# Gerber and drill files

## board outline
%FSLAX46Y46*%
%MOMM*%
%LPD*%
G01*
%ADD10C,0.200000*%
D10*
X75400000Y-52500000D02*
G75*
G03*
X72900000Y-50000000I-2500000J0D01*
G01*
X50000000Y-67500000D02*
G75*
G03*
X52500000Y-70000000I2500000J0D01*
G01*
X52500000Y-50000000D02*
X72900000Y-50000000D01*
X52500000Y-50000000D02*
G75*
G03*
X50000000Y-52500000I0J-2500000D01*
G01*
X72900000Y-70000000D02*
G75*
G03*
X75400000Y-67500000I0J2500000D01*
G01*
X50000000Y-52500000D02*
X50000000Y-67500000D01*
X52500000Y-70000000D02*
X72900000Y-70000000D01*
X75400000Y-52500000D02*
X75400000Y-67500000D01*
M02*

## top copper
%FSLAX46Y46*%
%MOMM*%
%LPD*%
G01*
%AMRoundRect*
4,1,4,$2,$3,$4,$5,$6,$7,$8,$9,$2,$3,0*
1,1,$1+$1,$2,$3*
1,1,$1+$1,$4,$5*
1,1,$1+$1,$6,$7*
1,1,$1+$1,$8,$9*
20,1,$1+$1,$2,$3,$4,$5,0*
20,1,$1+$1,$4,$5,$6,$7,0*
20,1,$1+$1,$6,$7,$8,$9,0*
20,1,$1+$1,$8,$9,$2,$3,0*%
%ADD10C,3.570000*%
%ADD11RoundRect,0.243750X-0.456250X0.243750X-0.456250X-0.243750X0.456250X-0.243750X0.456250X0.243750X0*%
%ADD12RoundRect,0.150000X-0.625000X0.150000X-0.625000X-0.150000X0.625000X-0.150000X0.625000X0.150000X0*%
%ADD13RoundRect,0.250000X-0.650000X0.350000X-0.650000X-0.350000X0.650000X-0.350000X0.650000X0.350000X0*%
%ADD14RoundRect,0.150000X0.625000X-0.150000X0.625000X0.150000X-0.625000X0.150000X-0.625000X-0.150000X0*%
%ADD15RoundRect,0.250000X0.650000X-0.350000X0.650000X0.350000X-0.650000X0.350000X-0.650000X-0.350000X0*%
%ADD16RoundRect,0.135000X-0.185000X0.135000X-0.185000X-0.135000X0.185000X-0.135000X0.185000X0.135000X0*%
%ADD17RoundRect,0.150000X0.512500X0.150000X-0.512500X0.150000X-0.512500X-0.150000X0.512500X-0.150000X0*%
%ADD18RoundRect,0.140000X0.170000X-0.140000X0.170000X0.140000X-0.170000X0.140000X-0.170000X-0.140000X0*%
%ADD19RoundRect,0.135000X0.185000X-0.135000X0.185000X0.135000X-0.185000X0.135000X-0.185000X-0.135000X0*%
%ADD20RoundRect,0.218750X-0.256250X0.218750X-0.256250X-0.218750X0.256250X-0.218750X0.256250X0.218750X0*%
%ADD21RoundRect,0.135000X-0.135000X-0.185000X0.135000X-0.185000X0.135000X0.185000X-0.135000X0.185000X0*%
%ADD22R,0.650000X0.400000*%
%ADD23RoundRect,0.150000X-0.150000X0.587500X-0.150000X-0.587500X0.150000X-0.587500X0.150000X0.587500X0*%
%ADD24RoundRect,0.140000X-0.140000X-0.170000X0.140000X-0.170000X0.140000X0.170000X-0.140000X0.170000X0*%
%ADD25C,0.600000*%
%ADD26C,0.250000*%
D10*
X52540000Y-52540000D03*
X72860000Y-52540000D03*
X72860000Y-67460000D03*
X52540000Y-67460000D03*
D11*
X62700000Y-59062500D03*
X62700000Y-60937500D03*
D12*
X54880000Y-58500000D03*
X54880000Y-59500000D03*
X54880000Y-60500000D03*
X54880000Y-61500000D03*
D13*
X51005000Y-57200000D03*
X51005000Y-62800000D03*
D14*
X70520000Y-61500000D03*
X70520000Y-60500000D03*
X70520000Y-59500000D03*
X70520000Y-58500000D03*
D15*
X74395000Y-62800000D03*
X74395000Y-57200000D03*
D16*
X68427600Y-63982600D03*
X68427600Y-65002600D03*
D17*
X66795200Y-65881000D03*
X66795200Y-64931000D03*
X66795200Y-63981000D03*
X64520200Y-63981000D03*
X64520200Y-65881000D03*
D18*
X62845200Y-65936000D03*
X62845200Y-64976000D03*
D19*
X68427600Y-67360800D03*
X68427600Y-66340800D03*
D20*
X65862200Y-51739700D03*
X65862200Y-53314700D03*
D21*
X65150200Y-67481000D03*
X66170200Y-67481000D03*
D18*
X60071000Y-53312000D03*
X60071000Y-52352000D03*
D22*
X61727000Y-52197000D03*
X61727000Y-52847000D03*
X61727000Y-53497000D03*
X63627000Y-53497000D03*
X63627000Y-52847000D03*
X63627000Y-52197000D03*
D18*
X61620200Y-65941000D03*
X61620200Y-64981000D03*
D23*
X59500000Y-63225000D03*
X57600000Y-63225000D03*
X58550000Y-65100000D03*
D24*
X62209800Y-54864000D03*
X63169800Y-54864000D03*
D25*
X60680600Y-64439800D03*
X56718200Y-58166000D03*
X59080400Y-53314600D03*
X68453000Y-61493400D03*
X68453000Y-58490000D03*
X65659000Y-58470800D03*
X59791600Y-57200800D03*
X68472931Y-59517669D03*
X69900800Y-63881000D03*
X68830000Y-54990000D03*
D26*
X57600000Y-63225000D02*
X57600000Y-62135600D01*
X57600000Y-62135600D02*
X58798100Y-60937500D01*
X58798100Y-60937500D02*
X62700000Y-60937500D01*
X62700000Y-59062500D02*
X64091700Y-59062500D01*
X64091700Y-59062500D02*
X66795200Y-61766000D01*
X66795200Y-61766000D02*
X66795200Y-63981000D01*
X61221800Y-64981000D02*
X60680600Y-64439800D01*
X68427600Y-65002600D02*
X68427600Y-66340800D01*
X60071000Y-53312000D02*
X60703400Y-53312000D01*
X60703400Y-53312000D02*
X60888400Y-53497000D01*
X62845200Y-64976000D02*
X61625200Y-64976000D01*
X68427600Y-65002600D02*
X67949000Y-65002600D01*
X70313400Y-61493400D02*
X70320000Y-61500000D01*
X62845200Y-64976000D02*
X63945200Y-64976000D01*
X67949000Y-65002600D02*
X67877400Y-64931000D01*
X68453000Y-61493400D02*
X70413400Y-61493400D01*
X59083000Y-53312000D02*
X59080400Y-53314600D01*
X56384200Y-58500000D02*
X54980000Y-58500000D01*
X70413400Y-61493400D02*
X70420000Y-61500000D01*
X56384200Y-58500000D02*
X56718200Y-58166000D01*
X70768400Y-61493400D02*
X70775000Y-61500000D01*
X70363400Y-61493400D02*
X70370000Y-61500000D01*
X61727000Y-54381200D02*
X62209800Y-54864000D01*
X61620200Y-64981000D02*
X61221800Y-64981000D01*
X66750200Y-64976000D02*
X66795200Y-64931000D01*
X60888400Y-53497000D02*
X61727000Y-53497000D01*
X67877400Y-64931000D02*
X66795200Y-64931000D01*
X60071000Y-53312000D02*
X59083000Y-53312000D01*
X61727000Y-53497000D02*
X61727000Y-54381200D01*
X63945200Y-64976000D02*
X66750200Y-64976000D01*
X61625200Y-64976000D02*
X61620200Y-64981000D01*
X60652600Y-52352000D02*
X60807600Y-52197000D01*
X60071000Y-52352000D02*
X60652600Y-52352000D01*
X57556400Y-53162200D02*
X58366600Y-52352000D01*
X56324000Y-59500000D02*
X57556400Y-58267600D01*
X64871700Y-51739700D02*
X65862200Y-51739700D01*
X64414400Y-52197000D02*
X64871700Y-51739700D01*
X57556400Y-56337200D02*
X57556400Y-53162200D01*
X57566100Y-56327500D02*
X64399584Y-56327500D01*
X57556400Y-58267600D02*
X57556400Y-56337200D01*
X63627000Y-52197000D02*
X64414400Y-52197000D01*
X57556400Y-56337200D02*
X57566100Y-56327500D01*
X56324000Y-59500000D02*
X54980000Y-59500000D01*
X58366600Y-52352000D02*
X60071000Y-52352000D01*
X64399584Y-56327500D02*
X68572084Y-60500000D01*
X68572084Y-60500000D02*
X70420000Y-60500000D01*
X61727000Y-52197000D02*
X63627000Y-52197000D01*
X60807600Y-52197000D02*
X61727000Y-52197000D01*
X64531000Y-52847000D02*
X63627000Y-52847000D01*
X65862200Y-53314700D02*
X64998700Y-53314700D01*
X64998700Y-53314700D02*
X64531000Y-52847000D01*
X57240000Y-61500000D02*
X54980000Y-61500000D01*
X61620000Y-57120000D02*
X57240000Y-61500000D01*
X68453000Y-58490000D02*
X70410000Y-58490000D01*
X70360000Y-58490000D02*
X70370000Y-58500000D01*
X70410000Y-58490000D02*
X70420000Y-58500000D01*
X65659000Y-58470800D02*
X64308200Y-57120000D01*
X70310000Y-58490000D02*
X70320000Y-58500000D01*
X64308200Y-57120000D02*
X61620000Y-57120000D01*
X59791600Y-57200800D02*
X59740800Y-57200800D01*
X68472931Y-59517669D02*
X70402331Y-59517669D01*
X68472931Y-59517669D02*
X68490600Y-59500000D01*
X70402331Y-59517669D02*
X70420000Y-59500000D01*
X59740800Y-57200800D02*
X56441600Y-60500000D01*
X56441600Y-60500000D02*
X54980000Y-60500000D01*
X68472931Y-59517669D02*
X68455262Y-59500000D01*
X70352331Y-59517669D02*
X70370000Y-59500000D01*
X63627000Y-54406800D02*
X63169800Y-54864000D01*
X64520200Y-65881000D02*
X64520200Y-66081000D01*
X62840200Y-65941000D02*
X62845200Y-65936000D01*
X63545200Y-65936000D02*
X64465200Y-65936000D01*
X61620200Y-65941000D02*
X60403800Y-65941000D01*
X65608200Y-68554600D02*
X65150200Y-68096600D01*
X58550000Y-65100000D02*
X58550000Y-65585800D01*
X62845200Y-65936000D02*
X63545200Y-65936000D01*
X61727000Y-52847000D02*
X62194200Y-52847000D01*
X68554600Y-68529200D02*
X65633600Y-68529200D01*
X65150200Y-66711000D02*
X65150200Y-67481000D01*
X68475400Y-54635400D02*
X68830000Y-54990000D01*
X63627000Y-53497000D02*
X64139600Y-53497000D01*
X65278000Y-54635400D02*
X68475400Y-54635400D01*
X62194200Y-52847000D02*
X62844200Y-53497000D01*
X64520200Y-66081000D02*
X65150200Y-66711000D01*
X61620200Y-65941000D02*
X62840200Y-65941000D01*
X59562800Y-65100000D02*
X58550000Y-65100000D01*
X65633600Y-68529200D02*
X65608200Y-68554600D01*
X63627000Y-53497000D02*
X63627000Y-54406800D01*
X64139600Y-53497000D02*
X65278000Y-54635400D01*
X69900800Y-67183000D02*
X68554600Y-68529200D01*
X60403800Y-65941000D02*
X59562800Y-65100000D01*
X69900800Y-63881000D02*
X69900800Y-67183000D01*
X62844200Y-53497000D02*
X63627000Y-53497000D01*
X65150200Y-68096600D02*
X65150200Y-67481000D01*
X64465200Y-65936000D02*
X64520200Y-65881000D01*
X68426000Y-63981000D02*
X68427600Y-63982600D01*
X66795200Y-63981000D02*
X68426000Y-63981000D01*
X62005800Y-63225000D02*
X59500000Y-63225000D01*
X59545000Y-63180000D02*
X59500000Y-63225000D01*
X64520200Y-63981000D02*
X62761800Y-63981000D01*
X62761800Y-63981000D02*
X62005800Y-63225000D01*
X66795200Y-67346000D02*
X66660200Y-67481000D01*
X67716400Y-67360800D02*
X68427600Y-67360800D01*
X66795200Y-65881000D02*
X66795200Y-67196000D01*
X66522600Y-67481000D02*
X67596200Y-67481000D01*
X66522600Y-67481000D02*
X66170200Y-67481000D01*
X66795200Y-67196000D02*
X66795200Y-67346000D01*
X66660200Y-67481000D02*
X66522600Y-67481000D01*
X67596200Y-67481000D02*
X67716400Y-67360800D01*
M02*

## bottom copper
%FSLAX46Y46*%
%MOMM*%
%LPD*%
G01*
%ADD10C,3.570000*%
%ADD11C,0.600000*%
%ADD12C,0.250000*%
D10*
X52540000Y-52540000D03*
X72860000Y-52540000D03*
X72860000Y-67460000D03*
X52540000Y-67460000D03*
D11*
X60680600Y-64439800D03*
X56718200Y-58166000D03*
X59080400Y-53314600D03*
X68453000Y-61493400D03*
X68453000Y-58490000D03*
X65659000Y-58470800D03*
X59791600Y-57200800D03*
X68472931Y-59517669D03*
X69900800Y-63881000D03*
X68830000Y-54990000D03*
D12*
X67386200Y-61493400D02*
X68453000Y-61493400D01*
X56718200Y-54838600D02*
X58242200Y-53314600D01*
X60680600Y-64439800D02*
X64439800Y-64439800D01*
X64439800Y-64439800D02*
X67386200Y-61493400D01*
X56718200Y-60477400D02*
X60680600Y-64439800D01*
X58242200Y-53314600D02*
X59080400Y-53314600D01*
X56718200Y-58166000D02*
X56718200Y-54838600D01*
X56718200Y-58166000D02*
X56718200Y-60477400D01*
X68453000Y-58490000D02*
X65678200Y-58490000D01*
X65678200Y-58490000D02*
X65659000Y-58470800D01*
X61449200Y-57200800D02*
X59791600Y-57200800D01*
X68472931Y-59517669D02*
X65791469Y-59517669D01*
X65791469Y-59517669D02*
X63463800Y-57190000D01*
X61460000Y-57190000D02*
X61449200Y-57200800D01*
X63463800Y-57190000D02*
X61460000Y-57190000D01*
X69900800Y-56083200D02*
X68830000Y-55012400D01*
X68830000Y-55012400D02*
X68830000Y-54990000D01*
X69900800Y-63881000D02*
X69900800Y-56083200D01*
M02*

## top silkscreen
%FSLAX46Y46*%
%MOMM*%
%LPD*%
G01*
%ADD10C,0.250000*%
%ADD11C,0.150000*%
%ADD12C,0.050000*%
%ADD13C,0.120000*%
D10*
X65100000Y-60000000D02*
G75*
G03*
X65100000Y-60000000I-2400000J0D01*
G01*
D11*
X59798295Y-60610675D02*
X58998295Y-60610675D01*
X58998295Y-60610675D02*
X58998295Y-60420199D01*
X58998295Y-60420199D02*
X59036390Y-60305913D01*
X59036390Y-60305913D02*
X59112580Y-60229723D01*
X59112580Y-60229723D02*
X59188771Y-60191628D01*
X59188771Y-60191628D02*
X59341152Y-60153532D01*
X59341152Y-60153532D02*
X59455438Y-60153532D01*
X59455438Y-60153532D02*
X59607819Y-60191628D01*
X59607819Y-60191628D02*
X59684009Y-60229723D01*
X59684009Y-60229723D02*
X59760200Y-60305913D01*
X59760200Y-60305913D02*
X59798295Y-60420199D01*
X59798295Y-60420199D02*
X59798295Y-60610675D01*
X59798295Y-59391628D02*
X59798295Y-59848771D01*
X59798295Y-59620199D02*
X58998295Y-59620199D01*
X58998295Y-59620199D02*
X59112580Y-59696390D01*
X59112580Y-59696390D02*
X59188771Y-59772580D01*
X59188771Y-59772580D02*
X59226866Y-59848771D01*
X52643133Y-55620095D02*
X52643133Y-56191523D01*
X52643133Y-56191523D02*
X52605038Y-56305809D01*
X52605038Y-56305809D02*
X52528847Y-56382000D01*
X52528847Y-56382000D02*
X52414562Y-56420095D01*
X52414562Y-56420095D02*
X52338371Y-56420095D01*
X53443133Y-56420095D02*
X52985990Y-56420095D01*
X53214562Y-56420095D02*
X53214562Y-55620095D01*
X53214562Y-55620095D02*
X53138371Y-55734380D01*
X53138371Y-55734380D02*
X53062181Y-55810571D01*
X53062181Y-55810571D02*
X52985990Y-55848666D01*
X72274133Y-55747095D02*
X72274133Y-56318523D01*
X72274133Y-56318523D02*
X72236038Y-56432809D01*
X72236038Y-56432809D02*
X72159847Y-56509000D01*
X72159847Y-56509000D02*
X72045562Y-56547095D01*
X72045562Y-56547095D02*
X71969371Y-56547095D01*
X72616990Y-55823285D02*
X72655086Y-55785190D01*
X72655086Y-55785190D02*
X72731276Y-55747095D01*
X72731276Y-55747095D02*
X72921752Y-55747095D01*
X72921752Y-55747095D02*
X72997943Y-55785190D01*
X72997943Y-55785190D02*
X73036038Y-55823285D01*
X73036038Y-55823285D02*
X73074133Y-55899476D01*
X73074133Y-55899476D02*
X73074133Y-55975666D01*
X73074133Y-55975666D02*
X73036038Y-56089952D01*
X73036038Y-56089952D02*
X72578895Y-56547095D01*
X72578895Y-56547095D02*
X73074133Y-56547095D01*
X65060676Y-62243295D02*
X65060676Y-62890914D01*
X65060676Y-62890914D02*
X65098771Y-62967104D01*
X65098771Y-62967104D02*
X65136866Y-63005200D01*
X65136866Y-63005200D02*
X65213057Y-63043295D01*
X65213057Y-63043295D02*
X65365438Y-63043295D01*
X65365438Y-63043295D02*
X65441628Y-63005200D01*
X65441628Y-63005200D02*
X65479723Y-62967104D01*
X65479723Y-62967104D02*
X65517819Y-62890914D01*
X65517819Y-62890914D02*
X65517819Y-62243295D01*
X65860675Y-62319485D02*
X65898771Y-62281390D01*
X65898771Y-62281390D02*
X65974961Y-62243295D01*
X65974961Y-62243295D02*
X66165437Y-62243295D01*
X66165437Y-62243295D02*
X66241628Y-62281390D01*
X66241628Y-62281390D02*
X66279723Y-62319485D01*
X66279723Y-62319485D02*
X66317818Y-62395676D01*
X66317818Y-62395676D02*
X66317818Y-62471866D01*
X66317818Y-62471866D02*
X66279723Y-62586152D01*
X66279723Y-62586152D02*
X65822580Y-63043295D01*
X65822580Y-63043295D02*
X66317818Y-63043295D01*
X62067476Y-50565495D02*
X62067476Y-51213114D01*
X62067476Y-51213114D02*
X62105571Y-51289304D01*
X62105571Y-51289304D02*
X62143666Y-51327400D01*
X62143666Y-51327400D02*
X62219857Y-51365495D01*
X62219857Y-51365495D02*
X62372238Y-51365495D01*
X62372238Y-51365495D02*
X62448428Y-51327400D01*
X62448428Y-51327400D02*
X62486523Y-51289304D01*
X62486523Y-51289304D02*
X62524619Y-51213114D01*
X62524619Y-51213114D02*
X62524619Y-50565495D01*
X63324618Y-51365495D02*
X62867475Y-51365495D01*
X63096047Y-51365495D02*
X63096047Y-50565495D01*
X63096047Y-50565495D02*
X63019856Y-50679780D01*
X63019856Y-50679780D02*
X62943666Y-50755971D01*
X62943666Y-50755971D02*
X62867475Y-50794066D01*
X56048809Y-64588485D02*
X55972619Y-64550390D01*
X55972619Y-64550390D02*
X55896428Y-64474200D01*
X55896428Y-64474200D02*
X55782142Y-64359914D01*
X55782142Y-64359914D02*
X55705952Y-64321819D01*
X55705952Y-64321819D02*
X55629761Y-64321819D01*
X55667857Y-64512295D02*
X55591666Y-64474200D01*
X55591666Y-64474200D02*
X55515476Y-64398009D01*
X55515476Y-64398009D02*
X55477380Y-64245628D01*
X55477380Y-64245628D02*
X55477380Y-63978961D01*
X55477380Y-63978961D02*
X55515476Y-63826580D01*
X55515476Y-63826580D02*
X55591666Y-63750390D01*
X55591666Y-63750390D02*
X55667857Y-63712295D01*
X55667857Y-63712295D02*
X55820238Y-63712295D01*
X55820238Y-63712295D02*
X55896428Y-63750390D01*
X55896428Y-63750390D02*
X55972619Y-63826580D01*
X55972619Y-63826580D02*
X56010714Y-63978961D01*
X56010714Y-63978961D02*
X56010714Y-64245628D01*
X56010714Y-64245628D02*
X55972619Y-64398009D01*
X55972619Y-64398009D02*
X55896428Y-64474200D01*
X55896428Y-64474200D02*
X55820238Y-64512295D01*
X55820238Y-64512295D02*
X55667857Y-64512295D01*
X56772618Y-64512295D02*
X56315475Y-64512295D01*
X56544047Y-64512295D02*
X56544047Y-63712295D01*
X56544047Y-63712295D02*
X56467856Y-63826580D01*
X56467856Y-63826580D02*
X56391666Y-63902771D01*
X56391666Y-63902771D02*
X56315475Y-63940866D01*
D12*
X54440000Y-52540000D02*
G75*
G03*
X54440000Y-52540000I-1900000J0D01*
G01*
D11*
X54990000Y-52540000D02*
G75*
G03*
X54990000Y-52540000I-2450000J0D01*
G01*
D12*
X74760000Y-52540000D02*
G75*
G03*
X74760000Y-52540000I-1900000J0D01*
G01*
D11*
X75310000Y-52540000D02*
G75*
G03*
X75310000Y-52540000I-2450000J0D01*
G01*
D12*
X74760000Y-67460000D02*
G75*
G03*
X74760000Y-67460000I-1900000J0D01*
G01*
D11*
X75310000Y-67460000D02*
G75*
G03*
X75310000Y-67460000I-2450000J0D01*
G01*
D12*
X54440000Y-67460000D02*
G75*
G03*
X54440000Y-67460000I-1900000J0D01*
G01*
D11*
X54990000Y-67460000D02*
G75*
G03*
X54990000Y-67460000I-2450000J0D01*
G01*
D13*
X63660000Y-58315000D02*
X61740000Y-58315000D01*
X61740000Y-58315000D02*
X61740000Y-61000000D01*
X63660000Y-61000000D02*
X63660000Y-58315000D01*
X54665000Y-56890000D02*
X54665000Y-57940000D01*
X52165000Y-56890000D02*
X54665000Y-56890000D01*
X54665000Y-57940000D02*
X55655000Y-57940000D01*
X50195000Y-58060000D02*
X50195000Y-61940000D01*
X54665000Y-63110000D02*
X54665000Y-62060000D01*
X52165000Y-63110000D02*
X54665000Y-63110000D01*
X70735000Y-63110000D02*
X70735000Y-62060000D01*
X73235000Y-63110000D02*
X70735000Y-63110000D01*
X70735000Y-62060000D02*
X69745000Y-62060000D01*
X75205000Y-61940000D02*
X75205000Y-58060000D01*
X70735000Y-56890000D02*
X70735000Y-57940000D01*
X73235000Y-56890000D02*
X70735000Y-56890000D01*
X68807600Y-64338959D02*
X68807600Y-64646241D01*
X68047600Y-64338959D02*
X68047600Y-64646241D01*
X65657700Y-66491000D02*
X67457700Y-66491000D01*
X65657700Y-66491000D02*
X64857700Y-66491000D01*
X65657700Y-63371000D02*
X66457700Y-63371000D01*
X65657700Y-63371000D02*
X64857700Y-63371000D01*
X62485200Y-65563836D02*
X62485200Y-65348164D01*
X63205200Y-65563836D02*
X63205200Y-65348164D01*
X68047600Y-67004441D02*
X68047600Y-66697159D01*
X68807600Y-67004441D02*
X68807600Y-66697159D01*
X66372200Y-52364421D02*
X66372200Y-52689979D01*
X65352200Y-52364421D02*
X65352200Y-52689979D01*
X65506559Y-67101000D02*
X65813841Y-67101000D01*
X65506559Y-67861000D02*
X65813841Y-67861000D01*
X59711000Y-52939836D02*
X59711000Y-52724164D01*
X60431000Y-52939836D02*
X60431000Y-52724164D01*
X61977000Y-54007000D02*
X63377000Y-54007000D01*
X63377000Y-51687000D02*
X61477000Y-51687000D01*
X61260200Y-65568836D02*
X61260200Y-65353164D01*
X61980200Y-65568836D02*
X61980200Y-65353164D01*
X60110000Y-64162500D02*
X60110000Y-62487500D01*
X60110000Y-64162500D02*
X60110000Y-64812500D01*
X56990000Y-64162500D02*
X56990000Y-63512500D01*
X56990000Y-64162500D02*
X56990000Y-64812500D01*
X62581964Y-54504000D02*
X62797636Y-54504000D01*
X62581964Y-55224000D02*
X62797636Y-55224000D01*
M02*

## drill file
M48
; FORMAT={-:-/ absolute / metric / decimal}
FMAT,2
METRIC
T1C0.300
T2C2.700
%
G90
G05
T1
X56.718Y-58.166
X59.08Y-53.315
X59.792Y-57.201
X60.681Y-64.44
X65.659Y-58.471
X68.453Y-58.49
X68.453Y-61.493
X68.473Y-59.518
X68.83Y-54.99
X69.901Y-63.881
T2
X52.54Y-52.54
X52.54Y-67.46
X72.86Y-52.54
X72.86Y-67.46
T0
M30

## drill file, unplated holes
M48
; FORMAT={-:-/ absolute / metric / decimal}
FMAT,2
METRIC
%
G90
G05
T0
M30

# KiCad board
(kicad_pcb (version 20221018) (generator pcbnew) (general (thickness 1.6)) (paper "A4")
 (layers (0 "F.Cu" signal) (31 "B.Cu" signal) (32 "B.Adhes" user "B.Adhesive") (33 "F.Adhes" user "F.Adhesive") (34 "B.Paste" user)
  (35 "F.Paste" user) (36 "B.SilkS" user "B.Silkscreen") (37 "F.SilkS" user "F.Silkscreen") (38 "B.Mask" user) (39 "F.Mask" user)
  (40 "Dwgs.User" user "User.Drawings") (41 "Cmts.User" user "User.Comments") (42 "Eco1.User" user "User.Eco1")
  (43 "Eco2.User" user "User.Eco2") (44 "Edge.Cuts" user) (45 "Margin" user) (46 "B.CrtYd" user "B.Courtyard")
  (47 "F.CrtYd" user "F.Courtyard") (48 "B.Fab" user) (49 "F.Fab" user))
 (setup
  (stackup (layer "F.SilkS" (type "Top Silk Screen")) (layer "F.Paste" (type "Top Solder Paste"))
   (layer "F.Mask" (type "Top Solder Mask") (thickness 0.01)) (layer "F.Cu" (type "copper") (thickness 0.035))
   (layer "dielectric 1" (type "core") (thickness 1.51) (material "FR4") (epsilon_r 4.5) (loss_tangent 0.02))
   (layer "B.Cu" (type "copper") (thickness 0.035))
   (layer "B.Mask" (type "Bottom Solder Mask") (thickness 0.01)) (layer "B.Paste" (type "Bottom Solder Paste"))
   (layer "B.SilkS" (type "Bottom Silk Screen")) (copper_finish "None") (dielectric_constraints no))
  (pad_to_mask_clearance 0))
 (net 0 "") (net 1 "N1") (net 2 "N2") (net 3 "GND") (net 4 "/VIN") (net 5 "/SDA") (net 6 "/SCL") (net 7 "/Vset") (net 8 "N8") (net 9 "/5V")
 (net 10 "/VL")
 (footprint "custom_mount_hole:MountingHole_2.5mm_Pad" (layer "F.Cu") (at 52.54 52.54)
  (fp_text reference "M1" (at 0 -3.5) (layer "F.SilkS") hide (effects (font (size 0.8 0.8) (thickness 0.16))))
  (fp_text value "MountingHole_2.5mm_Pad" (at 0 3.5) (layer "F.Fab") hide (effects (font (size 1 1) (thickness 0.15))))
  (fp_circle (center 0 0) (end 1.9 0) (stroke (width 0.05) (type solid)) (fill none) (layer "F.SilkS"))
  (fp_circle (center 0 0) (end 2.45 0) (stroke (width 0.15) (type solid)) (fill none) (layer "F.SilkS"))
  (pad "~" thru_hole circle (at 0 0) (size 3.57 3.57) (drill 2.7) (layers "*.Cu" "*.Mask")))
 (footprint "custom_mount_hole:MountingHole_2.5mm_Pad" (layer "F.Cu") (at 72.86 52.54)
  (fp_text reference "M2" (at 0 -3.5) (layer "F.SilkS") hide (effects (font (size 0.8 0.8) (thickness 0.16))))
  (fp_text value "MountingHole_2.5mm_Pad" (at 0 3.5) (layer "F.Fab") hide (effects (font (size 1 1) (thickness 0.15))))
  (fp_circle (center 0 0) (end 1.9 0) (stroke (width 0.05) (type solid)) (fill none) (layer "F.SilkS"))
  (fp_circle (center 0 0) (end 2.45 0) (stroke (width 0.15) (type solid)) (fill none) (layer "F.SilkS"))
  (pad "~" thru_hole circle (at 0 0) (size 3.57 3.57) (drill 2.7) (layers "*.Cu" "*.Mask")))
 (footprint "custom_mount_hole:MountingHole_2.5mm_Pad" (layer "F.Cu") (at 72.86 67.46)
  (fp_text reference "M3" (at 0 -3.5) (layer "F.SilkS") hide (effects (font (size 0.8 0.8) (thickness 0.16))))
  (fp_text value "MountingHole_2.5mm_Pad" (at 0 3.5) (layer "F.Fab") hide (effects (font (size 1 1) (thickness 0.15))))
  (fp_circle (center 0 0) (end 1.9 0) (stroke (width 0.05) (type solid)) (fill none) (layer "F.SilkS"))
  (fp_circle (center 0 0) (end 2.45 0) (stroke (width 0.15) (type solid)) (fill none) (layer "F.SilkS"))
  (pad "~" thru_hole circle (at 0 0) (size 3.57 3.57) (drill 2.7) (layers "*.Cu" "*.Mask")))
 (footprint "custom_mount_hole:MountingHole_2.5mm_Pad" (layer "F.Cu") (at 52.54 67.46)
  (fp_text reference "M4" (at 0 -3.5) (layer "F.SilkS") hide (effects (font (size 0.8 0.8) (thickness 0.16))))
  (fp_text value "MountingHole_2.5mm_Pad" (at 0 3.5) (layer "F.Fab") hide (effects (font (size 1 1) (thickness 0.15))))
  (fp_circle (center 0 0) (end 1.9 0) (stroke (width 0.05) (type solid)) (fill none) (layer "F.SilkS"))
  (fp_circle (center 0 0) (end 2.45 0) (stroke (width 0.15) (type solid)) (fill none) (layer "F.SilkS"))
  (pad "~" thru_hole circle (at 0 0) (size 3.57 3.57) (drill 2.7) (layers "*.Cu" "*.Mask")))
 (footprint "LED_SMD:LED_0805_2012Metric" (layer "F.Cu") (at 62.7 60 -90)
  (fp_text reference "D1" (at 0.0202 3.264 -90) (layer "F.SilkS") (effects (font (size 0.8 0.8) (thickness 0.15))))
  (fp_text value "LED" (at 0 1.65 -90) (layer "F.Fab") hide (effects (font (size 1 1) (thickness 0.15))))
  (fp_line (start -1.685 -0.96) (end -1.685 0.96) (stroke (width 0.12) (type solid)) (layer "F.SilkS"))
  (fp_line (start -1.685 0.96) (end 1 0.96) (stroke (width 0.12) (type solid)) (layer "F.SilkS"))
  (fp_line (start 1 -0.96) (end -1.685 -0.96) (stroke (width 0.12) (type solid)) (layer "F.SilkS"))
  (pad "1" smd roundrect (at -0.9375 0 270) (size 0.975 1.4) (layers "F.Cu" "F.Paste" "F.Mask") (roundrect_rratio 0.25) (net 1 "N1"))
  (pad "2" smd roundrect (at 0.9375 0 270) (size 0.975 1.4) (layers "F.Cu" "F.Paste" "F.Mask") (roundrect_rratio 0.25) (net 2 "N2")))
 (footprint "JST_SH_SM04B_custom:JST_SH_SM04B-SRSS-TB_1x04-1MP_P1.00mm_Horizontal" (layer "F.Cu") (at 52.88 60 -90)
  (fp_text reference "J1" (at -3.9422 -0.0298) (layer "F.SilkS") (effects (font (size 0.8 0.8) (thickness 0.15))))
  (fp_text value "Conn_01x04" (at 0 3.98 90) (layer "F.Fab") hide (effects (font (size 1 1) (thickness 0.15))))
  (fp_line (start -3.11 -1.785) (end -2.06 -1.785) (stroke (width 0.12) (type solid)) (layer "F.SilkS"))
  (fp_line (start -3.11 0.715) (end -3.11 -1.785) (stroke (width 0.12) (type solid)) (layer "F.SilkS"))
  (fp_line (start -2.06 -1.785) (end -2.06 -2.775) (stroke (width 0.12) (type solid)) (layer "F.SilkS"))
  (fp_line (start -1.94 2.685) (end 1.94 2.685) (stroke (width 0.12) (type solid)) (layer "F.SilkS"))
  (fp_line (start 3.11 -1.785) (end 2.06 -1.785) (stroke (width 0.12) (type solid)) (layer "F.SilkS"))
  (fp_line (start 3.11 0.715) (end 3.11 -1.785) (stroke (width 0.12) (type solid)) (layer "F.SilkS"))
  (pad "1" smd roundrect (at -1.5 -2 270) (size 0.6 1.55) (layers "F.Cu" "F.Paste" "F.Mask") (roundrect_rratio 0.25) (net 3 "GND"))
  (pad "2" smd roundrect (at -0.5 -2 270) (size 0.6 1.55) (layers "F.Cu" "F.Paste" "F.Mask") (roundrect_rratio 0.25) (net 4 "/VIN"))
  (pad "3" smd roundrect (at 0.5 -2 270) (size 0.6 1.55) (layers "F.Cu" "F.Paste" "F.Mask") (roundrect_rratio 0.25) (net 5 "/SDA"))
  (pad "4" smd roundrect (at 1.5 -2 270) (size 0.6 1.55) (layers "F.Cu" "F.Paste" "F.Mask") (roundrect_rratio 0.25) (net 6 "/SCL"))
  (pad "MP" smd roundrect (at -2.8 1.875 270) (size 1.2 1.8) (layers "F.Cu" "F.Paste" "F.Mask") (roundrect_rratio 0.2083333333))
  (pad "MP" smd roundrect (at 2.8 1.875 270) (size 1.2 1.8) (layers "F.Cu" "F.Paste" "F.Mask") (roundrect_rratio 0.2083333333)))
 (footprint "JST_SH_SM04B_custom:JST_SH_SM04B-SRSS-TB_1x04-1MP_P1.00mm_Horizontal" (layer "F.Cu") (at 72.52 60 90)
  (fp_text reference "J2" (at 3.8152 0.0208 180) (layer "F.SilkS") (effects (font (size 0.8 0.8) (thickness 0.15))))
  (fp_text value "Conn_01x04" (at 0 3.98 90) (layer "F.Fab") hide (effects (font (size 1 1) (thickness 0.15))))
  (fp_line (start -3.11 -1.785) (end -2.06 -1.785) (stroke (width 0.12) (type solid)) (layer "F.SilkS"))
  (fp_line (start -3.11 0.715) (end -3.11 -1.785) (stroke (width 0.12) (type solid)) (layer "F.SilkS"))
  (fp_line (start -2.06 -1.785) (end -2.06 -2.775) (stroke (width 0.12) (type solid)) (layer "F.SilkS"))
  (fp_line (start -1.94 2.685) (end 1.94 2.685) (stroke (width 0.12) (type solid)) (layer "F.SilkS"))
  (fp_line (start 3.11 -1.785) (end 2.06 -1.785) (stroke (width 0.12) (type solid)) (layer "F.SilkS"))
  (fp_line (start 3.11 0.715) (end 3.11 -1.785) (stroke (width 0.12) (type solid)) (layer "F.SilkS"))
  (pad "1" smd roundrect (at -1.5 -2 90) (size 0.6 1.55) (layers "F.Cu" "F.Paste" "F.Mask") (roundrect_rratio 0.25) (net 3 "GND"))
  (pad "2" smd roundrect (at -0.5 -2 90) (size 0.6 1.55) (layers "F.Cu" "F.Paste" "F.Mask") (roundrect_rratio 0.25) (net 4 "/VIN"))
  (pad "3" smd roundrect (at 0.5 -2 90) (size 0.6 1.55) (layers "F.Cu" "F.Paste" "F.Mask") (roundrect_rratio 0.25) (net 5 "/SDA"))
  (pad "4" smd roundrect (at 1.5 -2 90) (size 0.6 1.55) (layers "F.Cu" "F.Paste" "F.Mask") (roundrect_rratio 0.25) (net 6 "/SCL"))
  (pad "MP" smd roundrect (at -2.8 1.875 90) (size 1.2 1.8) (layers "F.Cu" "F.Paste" "F.Mask") (roundrect_rratio 0.2083333333))
  (pad "MP" smd roundrect (at 2.8 1.875 90) (size 1.2 1.8) (layers "F.Cu" "F.Paste" "F.Mask") (roundrect_rratio 0.2083333333)))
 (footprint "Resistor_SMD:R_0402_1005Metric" (layer "F.Cu") (at 68.4276 64.4926 -90)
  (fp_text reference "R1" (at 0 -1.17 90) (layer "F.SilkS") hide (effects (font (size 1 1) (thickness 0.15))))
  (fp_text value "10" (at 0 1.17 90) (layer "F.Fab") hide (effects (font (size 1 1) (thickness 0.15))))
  (fp_line (start -0.153641 -0.38) (end 0.153641 -0.38) (stroke (width 0.12) (type solid)) (layer "F.SilkS"))
  (fp_line (start -0.153641 0.38) (end 0.153641 0.38) (stroke (width 0.12) (type solid)) (layer "F.SilkS"))
  (pad "1" smd roundrect (at -0.51 0 270) (size 0.54 0.64) (layers "F.Cu" "F.Paste" "F.Mask") (roundrect_rratio 0.25) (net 1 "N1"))
  (pad "2" smd roundrect (at 0.51 0 270) (size 0.54 0.64) (layers "F.Cu" "F.Paste" "F.Mask") (roundrect_rratio 0.25) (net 3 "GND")))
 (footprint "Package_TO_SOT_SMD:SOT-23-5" (layer "F.Cu") (at 65.6577 64.931 180)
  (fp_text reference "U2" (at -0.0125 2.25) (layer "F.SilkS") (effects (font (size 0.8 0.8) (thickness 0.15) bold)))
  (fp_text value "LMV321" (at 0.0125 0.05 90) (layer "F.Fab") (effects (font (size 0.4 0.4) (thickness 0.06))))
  (fp_line (start 0 -1.56) (end -1.8 -1.56) (stroke (width 0.12) (type solid)) (layer "F.SilkS"))
  (fp_line (start 0 -1.56) (end 0.8 -1.56) (stroke (width 0.12) (type solid)) (layer "F.SilkS"))
  (fp_line (start 0 1.56) (end -0.8 1.56) (stroke (width 0.12) (type solid)) (layer "F.SilkS"))
  (fp_line (start 0 1.56) (end 0.8 1.56) (stroke (width 0.12) (type solid)) (layer "F.SilkS"))
  (pad "1" smd roundrect (at -1.1375 -0.95 180) (size 1.325 0.6) (layers "F.Cu" "F.Paste" "F.Mask") (roundrect_rratio 0.25) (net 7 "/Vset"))
  (pad "2" smd roundrect (at -1.1375 0 180) (size 1.325 0.6) (layers "F.Cu" "F.Paste" "F.Mask") (roundrect_rratio 0.25) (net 3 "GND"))
  (pad "3" smd roundrect (at -1.1375 0.95 180) (size 1.325 0.6) (layers "F.Cu" "F.Paste" "F.Mask") (roundrect_rratio 0.25) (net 1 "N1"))
  (pad "4" smd roundrect (at 1.1375 0.95 180) (size 1.325 0.6) (layers "F.Cu" "F.Paste" "F.Mask") (roundrect_rratio 0.25) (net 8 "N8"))
  (pad "5" smd roundrect (at 1.1375 -0.95 180) (size 1.325 0.6) (layers "F.Cu" "F.Paste" "F.Mask") (roundrect_rratio 0.25) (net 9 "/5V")))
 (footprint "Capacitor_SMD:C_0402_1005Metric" (layer "F.Cu") (at 62.8452 65.456 90)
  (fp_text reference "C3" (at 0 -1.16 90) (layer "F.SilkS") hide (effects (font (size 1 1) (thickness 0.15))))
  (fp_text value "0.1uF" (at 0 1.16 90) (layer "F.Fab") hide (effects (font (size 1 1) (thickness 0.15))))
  (fp_line (start -0.107836 -0.36) (end 0.107836 -0.36) (stroke (width 0.12) (type solid)) (layer "F.SilkS"))
  (fp_line (start -0.107836 0.36) (end 0.107836 0.36) (stroke (width 0.12) (type solid)) (layer "F.SilkS"))
  (pad "1" smd roundrect (at -0.48 0 90) (size 0.56 0.62) (layers "F.Cu" "F.Paste" "F.Mask") (roundrect_rratio 0.25) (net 9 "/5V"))
  (pad "2" smd roundrect (at 0.48 0 90) (size 0.56 0.62) (layers "F.Cu" "F.Paste" "F.Mask") (roundrect_rratio 0.25) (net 3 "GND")))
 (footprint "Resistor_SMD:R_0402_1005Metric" (layer "F.Cu") (at 68.4276 66.8508 90)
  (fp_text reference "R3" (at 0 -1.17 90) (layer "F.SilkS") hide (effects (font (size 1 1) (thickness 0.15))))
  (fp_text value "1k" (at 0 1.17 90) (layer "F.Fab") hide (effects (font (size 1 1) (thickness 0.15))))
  (fp_line (start -0.153641 -0.38) (end 0.153641 -0.38) (stroke (width 0.12) (type solid)) (layer "F.SilkS"))
  (fp_line (start -0.153641 0.38) (end 0.153641 0.38) (stroke (width 0.12) (type solid)) (layer "F.SilkS"))
  (pad "1" smd roundrect (at -0.51 0 90) (size 0.54 0.64) (layers "F.Cu" "F.Paste" "F.Mask") (roundrect_rratio 0.25) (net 7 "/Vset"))
  (pad "2" smd roundrect (at 0.51 0 90) (size 0.54 0.64) (layers "F.Cu" "F.Paste" "F.Mask") (roundrect_rratio 0.25) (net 3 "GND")))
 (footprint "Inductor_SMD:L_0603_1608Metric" (layer "F.Cu") (at 65.8622 52.5272 -90)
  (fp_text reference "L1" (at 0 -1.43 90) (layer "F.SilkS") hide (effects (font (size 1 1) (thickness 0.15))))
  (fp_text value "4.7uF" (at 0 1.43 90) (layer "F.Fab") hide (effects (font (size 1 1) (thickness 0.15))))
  (fp_line (start -0.162779 -0.51) (end 0.162779 -0.51) (stroke (width 0.12) (type solid)) (layer "F.SilkS"))
  (fp_line (start -0.162779 0.51) (end 0.162779 0.51) (stroke (width 0.12) (type solid)) (layer "F.SilkS"))
  (pad "1" smd roundrect (at -0.7875 0 270) (size 0.875 0.95) (layers "F.Cu" "F.Paste" "F.Mask") (roundrect_rratio 0.25) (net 4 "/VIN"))
  (pad "2" smd roundrect (at 0.7875 0 270) (size 0.875 0.95) (layers "F.Cu" "F.Paste" "F.Mask") (roundrect_rratio 0.25) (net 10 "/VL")))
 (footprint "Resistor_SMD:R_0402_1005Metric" (layer "F.Cu") (at 65.6602 67.481)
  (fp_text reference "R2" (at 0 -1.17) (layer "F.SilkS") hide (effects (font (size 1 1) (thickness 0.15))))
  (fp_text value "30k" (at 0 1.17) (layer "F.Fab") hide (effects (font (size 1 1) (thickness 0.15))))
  (fp_line (start -0.153641 -0.38) (end 0.153641 -0.38) (stroke (width 0.12) (type solid)) (layer "F.SilkS"))
  (fp_line (start -0.153641 0.38) (end 0.153641 0.38) (stroke (width 0.12) (type solid)) (layer "F.SilkS"))
  (pad "1" smd roundrect (at -0.51 0) (size 0.54 0.64) (layers "F.Cu" "F.Paste" "F.Mask") (roundrect_rratio 0.25) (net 9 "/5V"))
  (pad "2" smd roundrect (at 0.51 0) (size 0.54 0.64) (layers "F.Cu" "F.Paste" "F.Mask") (roundrect_rratio 0.25) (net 7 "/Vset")))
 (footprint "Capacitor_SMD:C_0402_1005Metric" (layer "F.Cu") (at 60.071 52.832 90)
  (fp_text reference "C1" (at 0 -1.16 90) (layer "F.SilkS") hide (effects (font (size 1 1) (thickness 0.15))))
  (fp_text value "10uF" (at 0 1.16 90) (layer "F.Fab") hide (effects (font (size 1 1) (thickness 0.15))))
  (fp_line (start -0.107836 -0.36) (end 0.107836 -0.36) (stroke (width 0.12) (type solid)) (layer "F.SilkS"))
  (fp_line (start -0.107836 0.36) (end 0.107836 0.36) (stroke (width 0.12) (type solid)) (layer "F.SilkS"))
  (pad "1" smd roundrect (at -0.48 0 90) (size 0.56 0.62) (layers "F.Cu" "F.Paste" "F.Mask") (roundrect_rratio 0.25) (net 3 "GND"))
  (pad "2" smd roundrect (at 0.48 0 90) (size 0.56 0.62) (layers "F.Cu" "F.Paste" "F.Mask") (roundrect_rratio 0.25) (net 4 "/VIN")))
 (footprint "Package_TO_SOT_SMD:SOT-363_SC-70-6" (layer "F.Cu") (at 62.677 52.847)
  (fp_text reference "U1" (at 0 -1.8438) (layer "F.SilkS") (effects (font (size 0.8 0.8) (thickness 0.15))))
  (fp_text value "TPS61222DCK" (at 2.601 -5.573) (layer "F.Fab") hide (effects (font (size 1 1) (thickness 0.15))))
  (fp_line (start -0.7 1.16) (end 0.7 1.16) (stroke (width 0.12) (type solid)) (layer "F.SilkS"))
  (fp_line (start 0.7 -1.16) (end -1.2 -1.16) (stroke (width 0.12) (type solid)) (layer "F.SilkS"))
  (pad "1" smd rect (at -0.95 -0.65) (size 0.65 0.4) (layers "F.Cu" "F.Paste" "F.Mask") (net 4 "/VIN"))
  (pad "2" smd rect (at -0.95 0) (size 0.65 0.4) (layers "F.Cu" "F.Paste" "F.Mask") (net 9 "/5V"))
  (pad "3" smd rect (at -0.95 0.65) (size 0.65 0.4) (layers "F.Cu" "F.Paste" "F.Mask") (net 3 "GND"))
  (pad "4" smd rect (at 0.95 0.65) (size 0.65 0.4) (layers "F.Cu" "F.Paste" "F.Mask") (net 9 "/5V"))
  (pad "5" smd rect (at 0.95 0) (size 0.65 0.4) (layers "F.Cu" "F.Paste" "F.Mask") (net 10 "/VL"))
  (pad "6" smd rect (at 0.95 -0.65) (size 0.65 0.4) (layers "F.Cu" "F.Paste" "F.Mask") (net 4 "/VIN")))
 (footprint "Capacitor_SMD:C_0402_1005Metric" (layer "F.Cu") (at 61.6202 65.461 90)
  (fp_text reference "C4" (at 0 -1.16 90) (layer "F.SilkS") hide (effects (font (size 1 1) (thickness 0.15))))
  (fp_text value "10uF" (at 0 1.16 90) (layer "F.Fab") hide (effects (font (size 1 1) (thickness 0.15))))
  (fp_line (start -0.107836 -0.36) (end 0.107836 -0.36) (stroke (width 0.12) (type solid)) (layer "F.SilkS"))
  (fp_line (start -0.107836 0.36) (end 0.107836 0.36) (stroke (width 0.12) (type solid)) (layer "F.SilkS"))
  (pad "1" smd roundrect (at -0.48 0 90) (size 0.56 0.62) (layers "F.Cu" "F.Paste" "F.Mask") (roundrect_rratio 0.25) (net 9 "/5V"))
  (pad "2" smd roundrect (at 0.48 0 90) (size 0.56 0.62) (layers "F.Cu" "F.Paste" "F.Mask") (roundrect_rratio 0.25) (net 3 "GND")))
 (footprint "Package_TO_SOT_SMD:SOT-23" (layer "F.Cu") (at 58.55 64.1625 -90)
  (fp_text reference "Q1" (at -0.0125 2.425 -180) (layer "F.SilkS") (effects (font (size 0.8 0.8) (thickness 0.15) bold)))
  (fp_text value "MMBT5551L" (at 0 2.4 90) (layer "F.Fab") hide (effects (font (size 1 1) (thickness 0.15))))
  (fp_line (start 0 -1.56) (end -1.675 -1.56) (stroke (width 0.12) (type solid)) (layer "F.SilkS"))
  (fp_line (start 0 -1.56) (end 0.65 -1.56) (stroke (width 0.12) (type solid)) (layer "F.SilkS"))
  (fp_line (start 0 1.56) (end -0.65 1.56) (stroke (width 0.12) (type solid)) (layer "F.SilkS"))
  (fp_line (start 0 1.56) (end 0.65 1.56) (stroke (width 0.12) (type solid)) (layer "F.SilkS"))
  (pad "1" smd roundrect (at -0.9375 -0.95 270) (size 1.475 0.6) (layers "F.Cu" "F.Paste" "F.Mask") (roundrect_rratio 0.25) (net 8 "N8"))
  (pad "2" smd roundrect (at -0.9375 0.95 270) (size 1.475 0.6) (layers "F.Cu" "F.Paste" "F.Mask") (roundrect_rratio 0.25) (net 2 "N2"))
  (pad "3" smd roundrect (at 0.9375 0 270) (size 1.475 0.6) (layers "F.Cu" "F.Paste" "F.Mask") (roundrect_rratio 0.25) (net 9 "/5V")))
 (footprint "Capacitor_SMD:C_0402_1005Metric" (layer "F.Cu") (at 62.6898 54.864)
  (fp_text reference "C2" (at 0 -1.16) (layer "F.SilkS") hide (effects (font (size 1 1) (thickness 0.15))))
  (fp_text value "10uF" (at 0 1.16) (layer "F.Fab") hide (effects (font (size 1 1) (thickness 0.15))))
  (fp_line (start -0.107836 -0.36) (end 0.107836 -0.36) (stroke (width 0.12) (type solid)) (layer "F.SilkS"))
  (fp_line (start -0.107836 0.36) (end 0.107836 0.36) (stroke (width 0.12) (type solid)) (layer "F.SilkS"))
  (pad "1" smd roundrect (at -0.48 0) (size 0.56 0.62) (layers "F.Cu" "F.Paste" "F.Mask") (roundrect_rratio 0.25) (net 3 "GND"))
  (pad "2" smd roundrect (at 0.48 0) (size 0.56 0.62) (layers "F.Cu" "F.Paste" "F.Mask") (roundrect_rratio 0.25) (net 9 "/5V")))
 (gr_circle (center 62.7 60) (end 65.1 60) (stroke (width 0.25) (type solid)) (fill none) (layer "F.SilkS"))
 (gr_arc (start 72.9 50) (mid 74.667767 50.732233) (end 75.4 52.5) (stroke (width 0.2) (type solid)) (layer "Edge.Cuts"))
 (gr_arc (start 52.5 70) (mid 50.732233 69.267767) (end 50 67.5) (stroke (width 0.2) (type solid)) (layer "Edge.Cuts"))
 (gr_line (start 52.5 50) (end 72.9 50) (stroke (width 0.2) (type solid)) (layer "Edge.Cuts"))
 (gr_arc (start 50 52.5) (mid 50.732233 50.732233) (end 52.5 50) (stroke (width 0.2) (type solid)) (layer "Edge.Cuts"))
 (gr_arc (start 75.4 67.5) (mid 74.667767 69.267767) (end 72.9 70) (stroke (width 0.2) (type solid)) (layer "Edge.Cuts"))
 (gr_line (start 50 52.5) (end 50 67.5) (stroke (width 0.2) (type solid)) (layer "Edge.Cuts"))
 (gr_line (start 52.5 70) (end 72.9 70) (stroke (width 0.2) (type solid)) (layer "Edge.Cuts"))
 (gr_line (start 75.4 52.5) (end 75.4 67.5) (stroke (width 0.2) (type solid)) (layer "Edge.Cuts"))
 (segment (start 61.2218 64.981) (end 60.6806 64.4398) (width 0.25) (layer "F.Cu") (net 3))
 (segment (start 68.4276 65.0026) (end 68.4276 66.3408) (width 0.25) (layer "F.Cu") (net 3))
 (segment (start 60.071 53.312) (end 60.7034 53.312) (width 0.25) (layer "F.Cu") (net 3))
 (segment (start 60.7034 53.312) (end 60.8884 53.497) (width 0.25) (layer "F.Cu") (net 3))
 (segment (start 62.8452 64.976) (end 61.6252 64.976) (width 0.25) (layer "F.Cu") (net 3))
 (segment (start 68.4276 65.0026) (end 67.949 65.0026) (width 0.25) (layer "F.Cu") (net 3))
 (segment (start 70.3134 61.4934) (end 70.32 61.5) (width 0.25) (layer "F.Cu") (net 3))
 (segment (start 62.8452 64.976) (end 63.9452 64.976) (width 0.25) (layer "F.Cu") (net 3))
 (segment (start 67.949 65.0026) (end 67.8774 64.931) (width 0.25) (layer "F.Cu") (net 3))
 (segment (start 68.453 61.4934) (end 70.4134 61.4934) (width 0.25) (layer "F.Cu") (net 3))
 (segment (start 59.083 53.312) (end 59.0804 53.3146) (width 0.25) (layer "F.Cu") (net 3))
 (segment (start 56.3842 58.5) (end 54.98 58.5) (width 0.25) (layer "F.Cu") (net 3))
 (segment (start 70.4134 61.4934) (end 70.42 61.5) (width 0.25) (layer "F.Cu") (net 3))
 (segment (start 56.3842 58.5) (end 56.7182 58.166) (width 0.25) (layer "F.Cu") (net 3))
 (segment (start 70.7684 61.4934) (end 70.775 61.5) (width 0.25) (layer "F.Cu") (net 3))
 (segment (start 70.3634 61.4934) (end 70.37 61.5) (width 0.25) (layer "F.Cu") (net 3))
 (segment (start 61.727 54.3812) (end 62.2098 54.864) (width 0.25) (layer "F.Cu") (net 3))
 (segment (start 61.6202 64.981) (end 61.2218 64.981) (width 0.25) (layer "F.Cu") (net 3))
 (segment (start 66.7502 64.976) (end 66.7952 64.931) (width 0.25) (layer "F.Cu") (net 3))
 (segment (start 60.8884 53.497) (end 61.727 53.497) (width 0.25) (layer "F.Cu") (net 3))
 (segment (start 67.8774 64.931) (end 66.7952 64.931) (width 0.25) (layer "F.Cu") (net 3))
 (segment (start 60.071 53.312) (end 59.083 53.312) (width 0.25) (layer "F.Cu") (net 3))
 (segment (start 61.727 53.497) (end 61.727 54.3812) (width 0.25) (layer "F.Cu") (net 3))
 (segment (start 63.9452 64.976) (end 66.7502 64.976) (width 0.25) (layer "F.Cu") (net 3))
 (segment (start 61.6252 64.976) (end 61.6202 64.981) (width 0.25) (layer "F.Cu") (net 3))
 (via (at 60.6806 64.4398) (size 0.6) (drill 0.3) (layers "F.Cu" "B.Cu") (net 3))
 (via (at 56.7182 58.166) (size 0.6) (drill 0.3) (layers "F.Cu" "B.Cu") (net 3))
 (via (at 59.0804 53.3146) (size 0.6) (drill 0.3) (layers "F.Cu" "B.Cu") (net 3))
 (via (at 68.453 61.4934) (size 0.6) (drill 0.3) (layers "F.Cu" "B.Cu") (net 3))
 (segment (start 67.3862 61.4934) (end 68.453 61.4934) (width 0.25) (layer "B.Cu") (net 3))
 (segment (start 56.7182 54.8386) (end 58.2422 53.3146) (width 0.25) (layer "B.Cu") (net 3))
 (segment (start 60.6806 64.4398) (end 64.4398 64.4398) (width 0.25) (layer "B.Cu") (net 3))
 (segment (start 64.4398 64.4398) (end 67.3862 61.4934) (width 0.25) (layer "B.Cu") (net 3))
 (segment (start 56.7182 60.4774) (end 60.6806 64.4398) (width 0.25) (layer "B.Cu") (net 3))
 (segment (start 58.2422 53.3146) (end 59.0804 53.3146) (width 0.25) (layer "B.Cu") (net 3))
 (segment (start 56.7182 58.166) (end 56.7182 54.8386) (width 0.25) (layer "B.Cu") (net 3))
 (segment (start 56.7182 58.166) (end 56.7182 60.4774) (width 0.25) (layer "B.Cu") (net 3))
 (segment (start 60.6526 52.352) (end 60.8076 52.197) (width 0.25) (layer "F.Cu") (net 4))
 (segment (start 60.071 52.352) (end 60.6526 52.352) (width 0.25) (layer "F.Cu") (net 4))
 (segment (start 57.5564 53.1622) (end 58.3666 52.352) (width 0.25) (layer "F.Cu") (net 4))
 (segment (start 56.324 59.5) (end 57.5564 58.2676) (width 0.25) (layer "F.Cu") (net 4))
 (segment (start 64.8717 51.7397) (end 65.8622 51.7397) (width 0.25) (layer "F.Cu") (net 4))
 (segment (start 64.4144 52.197) (end 64.8717 51.7397) (width 0.25) (layer "F.Cu") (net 4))
 (segment (start 57.5564 56.3372) (end 57.5564 53.1622) (width 0.25) (layer "F.Cu") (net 4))
 (segment (start 57.5661 56.3275) (end 64.399584 56.3275) (width 0.25) (layer "F.Cu") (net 4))
 (segment (start 57.5564 58.2676) (end 57.5564 56.3372) (width 0.25) (layer "F.Cu") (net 4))
 (segment (start 63.627 52.197) (end 64.4144 52.197) (width 0.25) (layer "F.Cu") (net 4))
 (segment (start 57.5564 56.3372) (end 57.5661 56.3275) (width 0.25) (layer "F.Cu") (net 4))
 (segment (start 56.324 59.5) (end 54.98 59.5) (width 0.25) (layer "F.Cu") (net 4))
 (segment (start 58.3666 52.352) (end 60.071 52.352) (width 0.25) (layer "F.Cu") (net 4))
 (segment (start 64.399584 56.3275) (end 68.572084 60.5) (width 0.25) (layer "F.Cu") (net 4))
 (segment (start 68.572084 60.5) (end 70.42 60.5) (width 0.25) (layer "F.Cu") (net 4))
 (segment (start 61.727 52.197) (end 63.627 52.197) (width 0.25) (layer "F.Cu") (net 4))
 (segment (start 60.8076 52.197) (end 61.727 52.197) (width 0.25) (layer "F.Cu") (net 4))
 (segment (start 64.531 52.847) (end 63.627 52.847) (width 0.25) (layer "F.Cu") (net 10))
 (segment (start 65.8622 53.3147) (end 64.9987 53.3147) (width 0.25) (layer "F.Cu") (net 10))
 (segment (start 64.9987 53.3147) (end 64.531 52.847) (width 0.25) (layer "F.Cu") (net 10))
 (segment (start 57.24 61.5) (end 54.98 61.5) (width 0.25) (layer "F.Cu") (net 6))
 (segment (start 61.62 57.12) (end 57.24 61.5) (width 0.25) (layer "F.Cu") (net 6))
 (segment (start 68.453 58.49) (end 70.41 58.49) (width 0.25) (layer "F.Cu") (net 6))
 (segment (start 70.36 58.49) (end 70.37 58.5) (width 0.25) (layer "F.Cu") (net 6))
 (segment (start 70.41 58.49) (end 70.42 58.5) (width 0.25) (layer "F.Cu") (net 6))
 (segment (start 65.659 58.4708) (end 64.3082 57.12) (width 0.25) (layer "F.Cu") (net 6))
 (segment (start 70.31 58.49) (end 70.32 58.5) (width 0.25) (layer "F.Cu") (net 6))
 (segment (start 64.3082 57.12) (end 61.62 57.12) (width 0.25) (layer "F.Cu") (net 6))
 (via (at 68.453 58.49) (size 0.6) (drill 0.3) (layers "F.Cu" "B.Cu") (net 6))
 (via (at 65.659 58.4708) (size 0.6) (drill 0.3) (layers "F.Cu" "B.Cu") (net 6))
 (segment (start 68.453 58.49) (end 65.6782 58.49) (width 0.25) (layer "B.Cu") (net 6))
 (segment (start 65.6782 58.49) (end 65.659 58.4708) (width 0.25) (layer "B.Cu") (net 6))
 (segment (start 59.7916 57.2008) (end 59.7408 57.2008) (width 0.25) (layer "F.Cu") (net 5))
 (segment (start 68.472931 59.517669) (end 70.402331 59.517669) (width 0.25) (layer "F.Cu") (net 5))
 (segment (start 68.472931 59.517669) (end 68.4906 59.5) (width 0.25) (layer "F.Cu") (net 5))
 (segment (start 70.402331 59.517669) (end 70.42 59.5) (width 0.25) (layer "F.Cu") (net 5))
 (segment (start 59.7408 57.2008) (end 56.4416 60.5) (width 0.25) (layer "F.Cu") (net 5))
 (segment (start 56.4416 60.5) (end 54.98 60.5) (width 0.25) (layer "F.Cu") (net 5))
 (segment (start 68.472931 59.517669) (end 68.455262 59.5) (width 0.25) (layer "F.Cu") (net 5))
 (segment (start 70.352331 59.517669) (end 70.37 59.5) (width 0.25) (layer "F.Cu") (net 5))
 (via (at 59.7916 57.2008) (size 0.6) (drill 0.3) (layers "F.Cu" "B.Cu") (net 5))
 (via (at 68.472931 59.517669) (size 0.6) (drill 0.3) (layers "F.Cu" "B.Cu") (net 5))
 (segment (start 61.4492 57.2008) (end 59.7916 57.2008) (width 0.25) (layer "B.Cu") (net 5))
 (segment (start 68.472931 59.517669) (end 65.791469 59.517669) (width 0.25) (layer "B.Cu") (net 5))
 (segment (start 65.791469 59.517669) (end 63.4638 57.19) (width 0.25) (layer "B.Cu") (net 5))
 (segment (start 61.46 57.19) (end 61.4492 57.2008) (width 0.25) (layer "B.Cu") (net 5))
 (segment (start 63.4638 57.19) (end 61.46 57.19) (width 0.25) (layer "B.Cu") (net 5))
 (segment (start 63.627 54.4068) (end 63.1698 54.864) (width 0.25) (layer "F.Cu") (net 9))
 (segment (start 64.5202 65.881) (end 64.5202 66.081) (width 0.25) (layer "F.Cu") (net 9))
 (segment (start 62.8402 65.941) (end 62.8452 65.936) (width 0.25) (layer "F.Cu") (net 9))
 (segment (start 63.5452 65.936) (end 64.4652 65.936) (width 0.25) (layer "F.Cu") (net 9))
 (segment (start 61.6202 65.941) (end 60.4038 65.941) (width 0.25) (layer "F.Cu") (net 9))
 (segment (start 65.6082 68.5546) (end 65.1502 68.0966) (width 0.25) (layer "F.Cu") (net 9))
 (segment (start 58.55 65.1) (end 58.55 65.5858) (width 0.25) (layer "F.Cu") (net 9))
 (segment (start 62.8452 65.936) (end 63.5452 65.936) (width 0.25) (layer "F.Cu") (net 9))
 (segment (start 61.727 52.847) (end 62.1942 52.847) (width 0.25) (layer "F.Cu") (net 9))
 (segment (start 68.5546 68.5292) (end 65.6336 68.5292) (width 0.25) (layer "F.Cu") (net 9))
 (segment (start 65.1502 66.711) (end 65.1502 67.481) (width 0.25) (layer "F.Cu") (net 9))
 (segment (start 68.4754 54.6354) (end 68.83 54.99) (width 0.25) (layer "F.Cu") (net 9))
 (segment (start 63.627 53.497) (end 64.1396 53.497) (width 0.25) (layer "F.Cu") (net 9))
 (segment (start 65.278 54.6354) (end 68.4754 54.6354) (width 0.25) (layer "F.Cu") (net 9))
 (segment (start 62.1942 52.847) (end 62.8442 53.497) (width 0.25) (layer "F.Cu") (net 9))
 (segment (start 64.5202 66.081) (end 65.1502 66.711) (width 0.25) (layer "F.Cu") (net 9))
 (segment (start 61.6202 65.941) (end 62.8402 65.941) (width 0.25) (layer "F.Cu") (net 9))
 (segment (start 59.5628 65.1) (end 58.55 65.1) (width 0.25) (layer "F.Cu") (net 9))
 (segment (start 65.6336 68.5292) (end 65.6082 68.5546) (width 0.25) (layer "F.Cu") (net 9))
 (segment (start 63.627 53.497) (end 63.627 54.4068) (width 0.25) (layer "F.Cu") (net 9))
 (segment (start 64.1396 53.497) (end 65.278 54.6354) (width 0.25) (layer "F.Cu") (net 9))
 (segment (start 69.9008 67.183) (end 68.5546 68.5292) (width 0.25) (layer "F.Cu") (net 9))
 (segment (start 60.4038 65.941) (end 59.5628 65.1) (width 0.25) (layer "F.Cu") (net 9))
 (segment (start 69.9008 63.881) (end 69.9008 67.183) (width 0.25) (layer "F.Cu") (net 9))
 (segment (start 62.8442 53.497) (end 63.627 53.497) (width 0.25) (layer "F.Cu") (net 9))
 (segment (start 65.1502 68.0966) (end 65.1502 67.481) (width 0.25) (layer "F.Cu") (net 9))
 (segment (start 64.4652 65.936) (end 64.5202 65.881) (width 0.25) (layer "F.Cu") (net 9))
 (via (at 69.9008 63.881) (size 0.6) (drill 0.3) (layers "F.Cu" "B.Cu") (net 9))
 (via (at 68.83 54.99) (size 0.6) (drill 0.3) (layers "F.Cu" "B.Cu") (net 9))
 (segment (start 69.9008 56.0832) (end 68.83 55.0124) (width 0.25) (layer "B.Cu") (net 9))
 (segment (start 68.83 55.0124) (end 68.83 54.99) (width 0.25) (layer "B.Cu") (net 9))
 (segment (start 69.9008 63.881) (end 69.9008 56.0832) (width 0.25) (layer "B.Cu") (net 9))
 (segment (start 68.426 63.981) (end 68.4276 63.9826) (width 0.25) (layer "F.Cu") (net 1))
 (segment (start 62.7 59.0625) (end 64.0917 59.0625) (width 0.25) (layer "F.Cu") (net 1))
 (segment (start 66.7952 61.766) (end 66.7952 63.981) (width 0.25) (layer "F.Cu") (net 1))
 (segment (start 66.7952 63.981) (end 68.426 63.981) (width 0.25) (layer "F.Cu") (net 1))
 (segment (start 64.0917 59.0625) (end 66.7952 61.766) (width 0.25) (layer "F.Cu") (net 1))
 (segment (start 58.7981 60.9375) (end 62.7 60.9375) (width 0.25) (layer "F.Cu") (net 2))
 (segment (start 57.6 63.225) (end 57.6 62.1356) (width 0.25) (layer "F.Cu") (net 2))
 (segment (start 57.6 62.1356) (end 58.7981 60.9375) (width 0.25) (layer "F.Cu") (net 2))
 (segment (start 62.0058 63.225) (end 59.5 63.225) (width 0.25) (layer "F.Cu") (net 8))
 (segment (start 59.545 63.18) (end 59.5 63.225) (width 0.25) (layer "F.Cu") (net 8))
 (segment (start 64.5202 63.981) (end 62.7618 63.981) (width 0.25) (layer "F.Cu") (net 8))
 (segment (start 62.7618 63.981) (end 62.0058 63.225) (width 0.25) (layer "F.Cu") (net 8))
 (segment (start 66.7952 67.346) (end 66.6602 67.481) (width 0.25) (layer "F.Cu") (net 7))
 (segment (start 67.7164 67.3608) (end 68.4276 67.3608) (width 0.25) (layer "F.Cu") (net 7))
 (segment (start 66.7952 65.881) (end 66.7952 67.196) (width 0.25) (layer "F.Cu") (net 7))
 (segment (start 66.5226 67.481) (end 67.5962 67.481) (width 0.25) (layer "F.Cu") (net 7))
 (segment (start 66.5226 67.481) (end 66.1702 67.481) (width 0.25) (layer "F.Cu") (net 7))
 (segment (start 66.7952 67.196) (end 66.7952 67.346) (width 0.25) (layer "F.Cu") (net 7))
 (segment (start 66.6602 67.481) (end 66.5226 67.481) (width 0.25) (layer "F.Cu") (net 7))
 (segment (start 67.5962 67.481) (end 67.7164 67.3608) (width 0.25) (layer "F.Cu") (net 7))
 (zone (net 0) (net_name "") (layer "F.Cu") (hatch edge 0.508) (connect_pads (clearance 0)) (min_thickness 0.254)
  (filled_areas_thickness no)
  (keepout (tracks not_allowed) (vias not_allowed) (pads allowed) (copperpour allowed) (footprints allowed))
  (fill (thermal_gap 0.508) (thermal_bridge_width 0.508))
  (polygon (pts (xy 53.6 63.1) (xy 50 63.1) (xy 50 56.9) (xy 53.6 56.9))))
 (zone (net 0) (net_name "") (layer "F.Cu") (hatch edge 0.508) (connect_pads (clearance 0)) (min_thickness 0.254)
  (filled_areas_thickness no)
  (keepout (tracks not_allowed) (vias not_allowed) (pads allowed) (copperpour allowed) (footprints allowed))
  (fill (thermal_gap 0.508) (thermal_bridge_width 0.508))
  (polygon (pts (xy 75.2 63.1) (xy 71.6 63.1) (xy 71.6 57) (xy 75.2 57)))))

